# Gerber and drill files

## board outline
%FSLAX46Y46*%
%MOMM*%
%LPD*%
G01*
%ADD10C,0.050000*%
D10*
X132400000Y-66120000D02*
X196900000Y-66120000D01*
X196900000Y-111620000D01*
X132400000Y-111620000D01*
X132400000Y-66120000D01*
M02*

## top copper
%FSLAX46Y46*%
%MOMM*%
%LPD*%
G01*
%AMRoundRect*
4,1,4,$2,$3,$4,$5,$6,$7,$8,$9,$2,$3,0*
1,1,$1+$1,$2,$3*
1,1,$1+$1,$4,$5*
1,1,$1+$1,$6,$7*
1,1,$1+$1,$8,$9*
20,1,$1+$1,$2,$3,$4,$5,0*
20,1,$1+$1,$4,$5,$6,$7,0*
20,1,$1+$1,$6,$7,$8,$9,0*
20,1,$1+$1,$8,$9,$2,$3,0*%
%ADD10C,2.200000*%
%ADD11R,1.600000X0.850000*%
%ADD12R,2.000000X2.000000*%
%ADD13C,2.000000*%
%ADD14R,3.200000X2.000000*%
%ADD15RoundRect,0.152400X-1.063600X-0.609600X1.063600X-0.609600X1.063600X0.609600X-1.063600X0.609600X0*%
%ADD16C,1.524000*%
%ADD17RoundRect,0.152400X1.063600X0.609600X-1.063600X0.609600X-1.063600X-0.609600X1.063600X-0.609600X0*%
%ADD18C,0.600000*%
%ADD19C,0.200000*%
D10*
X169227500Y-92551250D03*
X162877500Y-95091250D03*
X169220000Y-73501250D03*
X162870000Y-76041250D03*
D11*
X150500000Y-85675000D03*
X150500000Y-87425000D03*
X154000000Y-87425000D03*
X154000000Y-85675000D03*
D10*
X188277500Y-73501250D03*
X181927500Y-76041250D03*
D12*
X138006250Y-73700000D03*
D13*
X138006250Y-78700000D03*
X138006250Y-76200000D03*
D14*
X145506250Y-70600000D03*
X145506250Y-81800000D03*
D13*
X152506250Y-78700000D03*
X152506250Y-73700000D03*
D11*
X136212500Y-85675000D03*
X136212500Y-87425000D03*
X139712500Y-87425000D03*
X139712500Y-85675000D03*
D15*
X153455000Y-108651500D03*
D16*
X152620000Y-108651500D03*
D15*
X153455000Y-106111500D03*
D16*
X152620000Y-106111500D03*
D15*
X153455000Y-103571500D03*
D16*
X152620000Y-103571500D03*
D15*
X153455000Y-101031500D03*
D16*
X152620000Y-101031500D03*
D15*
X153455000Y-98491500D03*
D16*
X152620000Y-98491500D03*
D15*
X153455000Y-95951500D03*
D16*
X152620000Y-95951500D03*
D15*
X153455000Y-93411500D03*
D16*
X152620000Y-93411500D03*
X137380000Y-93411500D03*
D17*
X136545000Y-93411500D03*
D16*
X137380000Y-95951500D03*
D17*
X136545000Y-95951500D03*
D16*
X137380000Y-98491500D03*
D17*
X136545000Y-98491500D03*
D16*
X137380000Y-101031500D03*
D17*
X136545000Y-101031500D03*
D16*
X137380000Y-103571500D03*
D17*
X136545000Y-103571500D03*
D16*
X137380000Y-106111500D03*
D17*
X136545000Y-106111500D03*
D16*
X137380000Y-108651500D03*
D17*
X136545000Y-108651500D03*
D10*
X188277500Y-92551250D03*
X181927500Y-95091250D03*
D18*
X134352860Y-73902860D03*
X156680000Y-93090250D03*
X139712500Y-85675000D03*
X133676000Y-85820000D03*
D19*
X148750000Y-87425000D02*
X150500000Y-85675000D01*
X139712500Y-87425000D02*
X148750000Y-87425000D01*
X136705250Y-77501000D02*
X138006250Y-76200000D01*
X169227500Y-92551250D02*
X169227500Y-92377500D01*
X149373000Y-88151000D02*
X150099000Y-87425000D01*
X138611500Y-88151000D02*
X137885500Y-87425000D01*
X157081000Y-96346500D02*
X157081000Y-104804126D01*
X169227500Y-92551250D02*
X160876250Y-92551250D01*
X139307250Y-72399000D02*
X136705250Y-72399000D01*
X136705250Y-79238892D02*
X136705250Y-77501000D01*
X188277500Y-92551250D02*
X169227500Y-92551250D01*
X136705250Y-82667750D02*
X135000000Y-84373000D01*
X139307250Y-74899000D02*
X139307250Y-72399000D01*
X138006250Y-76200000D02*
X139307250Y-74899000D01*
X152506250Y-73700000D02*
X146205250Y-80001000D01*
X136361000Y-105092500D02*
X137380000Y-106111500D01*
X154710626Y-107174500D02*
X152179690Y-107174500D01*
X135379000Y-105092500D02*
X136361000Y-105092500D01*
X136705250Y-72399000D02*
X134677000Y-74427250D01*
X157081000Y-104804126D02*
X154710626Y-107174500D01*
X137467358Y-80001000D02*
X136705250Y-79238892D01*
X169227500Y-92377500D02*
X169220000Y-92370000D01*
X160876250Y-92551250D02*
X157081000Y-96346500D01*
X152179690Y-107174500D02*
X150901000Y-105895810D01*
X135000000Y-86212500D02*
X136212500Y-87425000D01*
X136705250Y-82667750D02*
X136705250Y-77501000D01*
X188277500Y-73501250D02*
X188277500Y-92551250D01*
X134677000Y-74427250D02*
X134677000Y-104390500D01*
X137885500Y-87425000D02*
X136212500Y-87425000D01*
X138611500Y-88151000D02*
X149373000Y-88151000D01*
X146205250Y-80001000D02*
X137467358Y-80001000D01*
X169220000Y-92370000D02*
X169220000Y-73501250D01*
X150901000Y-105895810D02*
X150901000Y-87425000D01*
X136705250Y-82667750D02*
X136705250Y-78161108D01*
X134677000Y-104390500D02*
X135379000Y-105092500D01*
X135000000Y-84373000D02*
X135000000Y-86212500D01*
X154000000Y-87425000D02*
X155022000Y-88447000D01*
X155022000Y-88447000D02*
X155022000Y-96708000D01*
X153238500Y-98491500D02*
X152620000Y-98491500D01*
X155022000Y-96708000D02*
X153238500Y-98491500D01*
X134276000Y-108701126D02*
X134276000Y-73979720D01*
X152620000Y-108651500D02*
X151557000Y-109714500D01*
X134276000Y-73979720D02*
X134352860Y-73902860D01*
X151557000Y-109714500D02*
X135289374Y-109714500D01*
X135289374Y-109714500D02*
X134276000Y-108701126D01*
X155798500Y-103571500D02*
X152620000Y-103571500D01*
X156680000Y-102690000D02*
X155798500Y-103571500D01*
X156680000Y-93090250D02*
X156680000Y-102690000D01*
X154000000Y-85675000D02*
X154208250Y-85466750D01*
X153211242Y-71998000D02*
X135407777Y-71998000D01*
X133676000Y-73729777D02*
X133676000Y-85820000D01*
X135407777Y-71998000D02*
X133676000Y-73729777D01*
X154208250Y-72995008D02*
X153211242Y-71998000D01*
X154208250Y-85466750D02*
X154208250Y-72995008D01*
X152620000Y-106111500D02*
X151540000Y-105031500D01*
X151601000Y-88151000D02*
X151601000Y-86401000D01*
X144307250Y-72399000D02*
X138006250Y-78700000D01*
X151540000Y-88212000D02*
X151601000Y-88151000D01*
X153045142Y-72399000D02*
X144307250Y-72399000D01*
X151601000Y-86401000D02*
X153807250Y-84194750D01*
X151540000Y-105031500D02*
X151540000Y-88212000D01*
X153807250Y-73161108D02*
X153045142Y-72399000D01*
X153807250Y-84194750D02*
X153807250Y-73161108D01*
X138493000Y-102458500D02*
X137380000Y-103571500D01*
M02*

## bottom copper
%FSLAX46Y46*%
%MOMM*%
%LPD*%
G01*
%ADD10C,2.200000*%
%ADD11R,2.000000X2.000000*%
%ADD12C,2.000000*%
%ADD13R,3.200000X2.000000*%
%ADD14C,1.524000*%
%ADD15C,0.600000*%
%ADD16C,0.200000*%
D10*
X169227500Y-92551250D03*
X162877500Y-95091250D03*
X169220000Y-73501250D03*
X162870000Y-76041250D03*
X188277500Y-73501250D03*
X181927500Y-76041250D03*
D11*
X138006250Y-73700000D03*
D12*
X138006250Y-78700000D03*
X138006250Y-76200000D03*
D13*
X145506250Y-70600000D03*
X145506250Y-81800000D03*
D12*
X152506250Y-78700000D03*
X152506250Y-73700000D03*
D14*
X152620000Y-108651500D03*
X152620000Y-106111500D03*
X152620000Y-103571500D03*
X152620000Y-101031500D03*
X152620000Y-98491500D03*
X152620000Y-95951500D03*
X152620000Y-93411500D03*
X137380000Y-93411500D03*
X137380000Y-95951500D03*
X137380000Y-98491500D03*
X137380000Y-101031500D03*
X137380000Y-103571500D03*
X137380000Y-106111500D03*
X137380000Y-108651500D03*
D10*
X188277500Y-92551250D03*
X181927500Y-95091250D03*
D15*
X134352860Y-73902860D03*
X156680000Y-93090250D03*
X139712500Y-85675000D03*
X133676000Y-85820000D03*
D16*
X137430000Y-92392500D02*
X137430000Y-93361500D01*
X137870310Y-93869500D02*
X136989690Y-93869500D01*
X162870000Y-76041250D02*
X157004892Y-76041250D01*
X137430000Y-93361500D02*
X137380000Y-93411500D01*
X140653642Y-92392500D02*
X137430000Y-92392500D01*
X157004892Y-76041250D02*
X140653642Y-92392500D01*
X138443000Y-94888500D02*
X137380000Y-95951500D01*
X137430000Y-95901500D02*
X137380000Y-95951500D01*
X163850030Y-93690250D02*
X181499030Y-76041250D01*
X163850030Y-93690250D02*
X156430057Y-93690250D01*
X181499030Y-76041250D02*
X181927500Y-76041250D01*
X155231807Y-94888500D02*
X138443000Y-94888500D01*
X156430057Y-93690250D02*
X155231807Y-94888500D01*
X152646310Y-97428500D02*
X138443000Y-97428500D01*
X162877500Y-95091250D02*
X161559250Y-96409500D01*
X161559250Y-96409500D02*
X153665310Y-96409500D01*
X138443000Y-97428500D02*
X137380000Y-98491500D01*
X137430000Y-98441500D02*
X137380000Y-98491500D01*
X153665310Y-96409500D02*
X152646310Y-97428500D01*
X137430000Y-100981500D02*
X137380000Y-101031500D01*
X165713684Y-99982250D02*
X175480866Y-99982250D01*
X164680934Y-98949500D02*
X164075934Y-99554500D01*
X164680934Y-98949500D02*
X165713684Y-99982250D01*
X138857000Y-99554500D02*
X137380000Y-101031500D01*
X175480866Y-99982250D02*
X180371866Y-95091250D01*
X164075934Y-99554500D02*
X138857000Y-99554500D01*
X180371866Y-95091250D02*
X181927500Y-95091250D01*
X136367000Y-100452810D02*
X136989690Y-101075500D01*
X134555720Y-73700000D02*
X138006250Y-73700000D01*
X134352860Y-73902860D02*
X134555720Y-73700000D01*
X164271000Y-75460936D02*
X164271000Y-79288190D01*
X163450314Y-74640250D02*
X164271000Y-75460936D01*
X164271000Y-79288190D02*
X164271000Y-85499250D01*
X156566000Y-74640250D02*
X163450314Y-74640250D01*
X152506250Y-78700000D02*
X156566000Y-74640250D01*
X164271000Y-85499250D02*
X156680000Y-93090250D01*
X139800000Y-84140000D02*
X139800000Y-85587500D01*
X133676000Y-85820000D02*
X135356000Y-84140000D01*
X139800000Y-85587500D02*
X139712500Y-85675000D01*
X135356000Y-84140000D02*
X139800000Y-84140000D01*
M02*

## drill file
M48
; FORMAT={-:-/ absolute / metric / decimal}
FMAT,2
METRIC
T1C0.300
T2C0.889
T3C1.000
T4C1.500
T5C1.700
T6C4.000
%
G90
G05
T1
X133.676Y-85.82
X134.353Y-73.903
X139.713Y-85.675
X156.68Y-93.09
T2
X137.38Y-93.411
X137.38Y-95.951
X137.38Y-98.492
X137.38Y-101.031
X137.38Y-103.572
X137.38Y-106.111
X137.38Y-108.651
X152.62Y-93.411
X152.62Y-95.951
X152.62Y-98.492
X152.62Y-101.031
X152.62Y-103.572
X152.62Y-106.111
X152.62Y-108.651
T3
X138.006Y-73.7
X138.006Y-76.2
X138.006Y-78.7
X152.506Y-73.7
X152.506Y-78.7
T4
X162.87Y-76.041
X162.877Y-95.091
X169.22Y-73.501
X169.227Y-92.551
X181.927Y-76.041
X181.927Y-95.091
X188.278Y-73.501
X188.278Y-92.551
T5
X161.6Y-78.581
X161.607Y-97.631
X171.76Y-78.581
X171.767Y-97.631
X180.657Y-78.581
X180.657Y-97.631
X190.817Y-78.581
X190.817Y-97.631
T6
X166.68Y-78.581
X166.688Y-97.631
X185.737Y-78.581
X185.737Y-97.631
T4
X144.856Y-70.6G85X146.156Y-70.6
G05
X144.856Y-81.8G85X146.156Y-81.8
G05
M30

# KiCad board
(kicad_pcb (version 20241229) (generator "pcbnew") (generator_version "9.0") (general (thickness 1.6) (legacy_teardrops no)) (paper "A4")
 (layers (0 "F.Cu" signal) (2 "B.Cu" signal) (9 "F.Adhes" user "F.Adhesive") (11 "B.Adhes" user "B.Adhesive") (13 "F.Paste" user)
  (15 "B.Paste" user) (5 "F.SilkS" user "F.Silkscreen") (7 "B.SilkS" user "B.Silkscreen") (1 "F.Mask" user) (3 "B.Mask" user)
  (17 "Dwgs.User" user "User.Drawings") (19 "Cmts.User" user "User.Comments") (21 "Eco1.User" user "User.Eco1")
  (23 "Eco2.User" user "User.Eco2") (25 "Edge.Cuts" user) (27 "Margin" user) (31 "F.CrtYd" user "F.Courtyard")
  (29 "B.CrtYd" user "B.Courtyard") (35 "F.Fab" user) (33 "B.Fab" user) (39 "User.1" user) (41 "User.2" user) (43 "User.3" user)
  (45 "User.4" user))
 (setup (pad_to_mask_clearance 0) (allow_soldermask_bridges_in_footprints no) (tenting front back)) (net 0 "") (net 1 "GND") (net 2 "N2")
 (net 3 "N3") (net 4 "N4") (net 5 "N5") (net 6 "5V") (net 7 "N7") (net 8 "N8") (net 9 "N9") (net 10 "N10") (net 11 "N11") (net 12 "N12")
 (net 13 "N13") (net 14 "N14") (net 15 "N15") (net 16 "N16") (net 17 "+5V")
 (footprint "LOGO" (layer "F.Cu") (at 140.493481 67.83475)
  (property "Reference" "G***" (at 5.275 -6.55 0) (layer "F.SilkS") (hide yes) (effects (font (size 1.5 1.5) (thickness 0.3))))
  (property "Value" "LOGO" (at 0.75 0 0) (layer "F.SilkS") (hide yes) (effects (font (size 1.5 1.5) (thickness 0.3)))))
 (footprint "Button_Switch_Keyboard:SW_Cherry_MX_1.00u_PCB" (layer "F.Cu") (at 169.2275 92.55125)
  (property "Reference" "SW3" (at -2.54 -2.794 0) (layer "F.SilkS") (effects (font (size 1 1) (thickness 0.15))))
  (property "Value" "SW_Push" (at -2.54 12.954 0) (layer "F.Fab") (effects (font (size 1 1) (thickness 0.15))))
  (pad "" np_thru_hole circle (at -7.62 5.08) (size 1.7 1.7) (drill 1.7) (layers "*.Cu" "*.Mask"))
  (pad "" np_thru_hole circle (at -2.54 5.08) (size 4 4) (drill 4) (layers "*.Cu" "*.Mask"))
  (pad "" np_thru_hole circle (at 2.54 5.08) (size 1.7 1.7) (drill 1.7) (layers "*.Cu" "*.Mask"))
  (pad "1" thru_hole circle (at 0 0) (size 2.2 2.2) (drill 1.5) (layers "*.Cu" "*.Mask") (remove_unused_layers no) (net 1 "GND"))
  (pad "2" thru_hole circle (at -6.35 2.54) (size 2.2 2.2) (drill 1.5) (layers "*.Cu" "*.Mask") (remove_unused_layers no) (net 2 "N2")))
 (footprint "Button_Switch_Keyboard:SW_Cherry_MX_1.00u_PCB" (layer "F.Cu") (at 169.22 73.50125)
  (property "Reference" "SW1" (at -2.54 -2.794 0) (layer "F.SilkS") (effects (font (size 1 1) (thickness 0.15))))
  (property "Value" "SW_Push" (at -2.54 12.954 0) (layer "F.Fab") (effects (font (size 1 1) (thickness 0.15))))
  (pad "" np_thru_hole circle (at -7.62 5.08) (size 1.7 1.7) (drill 1.7) (layers "*.Cu" "*.Mask"))
  (pad "" np_thru_hole circle (at -2.54 5.08) (size 4 4) (drill 4) (layers "*.Cu" "*.Mask"))
  (pad "" np_thru_hole circle (at 2.54 5.08) (size 1.7 1.7) (drill 1.7) (layers "*.Cu" "*.Mask"))
  (pad "1" thru_hole circle (at 0 0) (size 2.2 2.2) (drill 1.5) (layers "*.Cu" "*.Mask") (remove_unused_layers no) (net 1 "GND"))
  (pad "2" thru_hole circle (at -6.35 2.54) (size 2.2 2.2) (drill 1.5) (layers "*.Cu" "*.Mask") (remove_unused_layers no) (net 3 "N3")))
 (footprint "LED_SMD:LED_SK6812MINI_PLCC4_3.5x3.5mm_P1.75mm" (layer "F.Cu") (at 152.25 86.55)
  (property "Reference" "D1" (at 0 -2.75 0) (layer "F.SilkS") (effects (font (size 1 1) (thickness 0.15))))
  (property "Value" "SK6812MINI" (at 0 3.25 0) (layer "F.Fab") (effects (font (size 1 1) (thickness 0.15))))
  (pad "1" smd rect (at -1.75 -0.875) (size 1.6 0.85) (layers "F.Cu" "F.Mask" "F.Paste") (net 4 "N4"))
  (pad "2" smd rect (at -1.75 0.875) (size 1.6 0.85) (layers "F.Cu" "F.Mask" "F.Paste") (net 1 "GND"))
  (pad "3" smd rect (at 1.75 0.875) (size 1.6 0.85) (layers "F.Cu" "F.Mask" "F.Paste") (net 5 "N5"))
  (pad "4" smd rect (at 1.75 -0.875) (size 1.6 0.85) (layers "F.Cu" "F.Mask" "F.Paste") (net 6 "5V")))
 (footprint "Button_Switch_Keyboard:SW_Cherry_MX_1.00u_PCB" (layer "F.Cu") (at 188.2775 73.50125)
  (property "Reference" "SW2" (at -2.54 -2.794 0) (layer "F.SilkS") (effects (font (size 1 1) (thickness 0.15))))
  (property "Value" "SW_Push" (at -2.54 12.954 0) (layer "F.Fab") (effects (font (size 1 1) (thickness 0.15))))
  (pad "" np_thru_hole circle (at -7.62 5.08) (size 1.7 1.7) (drill 1.7) (layers "*.Cu" "*.Mask"))
  (pad "" np_thru_hole circle (at -2.54 5.08) (size 4 4) (drill 4) (layers "*.Cu" "*.Mask"))
  (pad "" np_thru_hole circle (at 2.54 5.08) (size 1.7 1.7) (drill 1.7) (layers "*.Cu" "*.Mask"))
  (pad "1" thru_hole circle (at 0 0) (size 2.2 2.2) (drill 1.5) (layers "*.Cu" "*.Mask") (remove_unused_layers no) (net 1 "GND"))
  (pad "2" thru_hole circle (at -6.35 2.54) (size 2.2 2.2) (drill 1.5) (layers "*.Cu" "*.Mask") (remove_unused_layers no) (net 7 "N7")))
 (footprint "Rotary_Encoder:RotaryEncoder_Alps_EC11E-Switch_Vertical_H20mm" (layer "F.Cu") (at 138.00625 73.7)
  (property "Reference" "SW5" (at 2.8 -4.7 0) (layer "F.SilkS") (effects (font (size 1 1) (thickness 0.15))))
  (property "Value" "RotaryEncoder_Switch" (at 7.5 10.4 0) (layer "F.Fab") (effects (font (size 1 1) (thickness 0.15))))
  (pad "A" thru_hole rect (at 0 0) (size 2 2) (drill 1) (layers "*.Cu" "*.Mask") (remove_unused_layers no) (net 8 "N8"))
  (pad "B" thru_hole circle (at 0 5) (size 2 2) (drill 1) (layers "*.Cu" "*.Mask") (remove_unused_layers no) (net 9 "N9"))
  (pad "C" thru_hole circle (at 0 2.5) (size 2 2) (drill 1) (layers "*.Cu" "*.Mask") (remove_unused_layers no) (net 1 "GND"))
  (pad "MP" thru_hole rect (at 7.5 -3.1) (size 3.2 2) (drill oval 2.8 1.5) (layers "*.Cu" "*.Mask") (remove_unused_layers no))
  (pad "MP" thru_hole rect (at 7.5 8.1) (size 3.2 2) (drill oval 2.8 1.5) (layers "*.Cu" "*.Mask") (remove_unused_layers no))
  (pad "S1" thru_hole circle (at 14.5 5) (size 2 2) (drill 1) (layers "*.Cu" "*.Mask") (remove_unused_layers no) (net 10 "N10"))
  (pad "S2" thru_hole circle (at 14.5 0) (size 2 2) (drill 1) (layers "*.Cu" "*.Mask") (remove_unused_layers no) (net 1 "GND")))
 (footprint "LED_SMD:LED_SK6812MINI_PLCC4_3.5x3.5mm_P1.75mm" (layer "F.Cu") (at 137.9625 86.55)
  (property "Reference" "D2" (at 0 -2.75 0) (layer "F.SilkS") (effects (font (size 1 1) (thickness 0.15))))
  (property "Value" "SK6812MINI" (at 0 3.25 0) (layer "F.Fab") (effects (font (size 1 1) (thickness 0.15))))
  (pad "1" smd rect (at -1.75 -0.875) (size 1.6 0.85) (layers "F.Cu" "F.Mask" "F.Paste") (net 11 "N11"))
  (pad "2" smd rect (at -1.75 0.875) (size 1.6 0.85) (layers "F.Cu" "F.Mask" "F.Paste") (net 1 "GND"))
  (pad "3" smd rect (at 1.75 0.875) (size 1.6 0.85) (layers "F.Cu" "F.Mask" "F.Paste") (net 4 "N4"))
  (pad "4" smd rect (at 1.75 -0.875) (size 1.6 0.85) (layers "F.Cu" "F.Mask" "F.Paste") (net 6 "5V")))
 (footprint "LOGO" (layer "F.Cu") (at 189.413481 67.69475)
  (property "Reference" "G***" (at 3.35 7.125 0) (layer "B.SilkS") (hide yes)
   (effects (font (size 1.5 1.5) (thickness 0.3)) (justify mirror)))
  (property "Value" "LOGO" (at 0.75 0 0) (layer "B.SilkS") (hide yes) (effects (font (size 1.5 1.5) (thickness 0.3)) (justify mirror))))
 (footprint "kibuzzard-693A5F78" (layer "F.Cu") (at 176.275 108.05 180)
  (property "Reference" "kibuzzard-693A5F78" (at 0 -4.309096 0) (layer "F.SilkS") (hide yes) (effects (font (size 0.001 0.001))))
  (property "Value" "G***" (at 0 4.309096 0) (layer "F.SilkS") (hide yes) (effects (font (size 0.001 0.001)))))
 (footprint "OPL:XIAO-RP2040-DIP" (layer "F.Cu") (at 145 101.0315 180)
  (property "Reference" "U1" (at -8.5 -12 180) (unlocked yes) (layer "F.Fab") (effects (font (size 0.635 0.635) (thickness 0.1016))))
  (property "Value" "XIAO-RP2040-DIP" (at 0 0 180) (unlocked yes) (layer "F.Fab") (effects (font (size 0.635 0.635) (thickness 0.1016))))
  (pad "1" smd roundrect (at -8.455 -7.62) (size 2.432 1.524) (layers "F.Cu" "F.Mask") (roundrect_rratio 0.1) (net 8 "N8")
   (thermal_bridge_angle 45))
  (pad "1" thru_hole circle (at -7.62 -7.62) (size 1.524 1.524) (drill 0.889) (layers "*.Cu" "*.Mask") (remove_unused_layers no)
   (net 8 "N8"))
  (pad "2" smd roundrect (at -8.455 -5.08) (size 2.432 1.524) (layers "F.Cu" "F.Mask") (roundrect_rratio 0.1) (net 9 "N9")
   (thermal_bridge_angle 45))
  (pad "2" thru_hole circle (at -7.62 -5.08) (size 1.524 1.524) (drill 0.889) (layers "*.Cu" "*.Mask") (remove_unused_layers no)
   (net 9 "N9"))
  (pad "3" smd roundrect (at -8.455 -2.54) (size 2.432 1.524) (layers "F.Cu" "F.Mask") (roundrect_rratio 0.1) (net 10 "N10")
   (thermal_bridge_angle 45))
  (pad "3" thru_hole circle (at -7.62 -2.54) (size 1.524 1.524) (drill 0.889) (layers "*.Cu" "*.Mask") (remove_unused_layers no)
   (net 10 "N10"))
  (pad "4" smd roundrect (at -8.455 0) (size 2.432 1.524) (layers "F.Cu" "F.Mask") (roundrect_rratio 0.1) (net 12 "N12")
   (thermal_bridge_angle 45))
  (pad "4" thru_hole circle (at -7.62 0) (size 1.524 1.524) (drill 0.889) (layers "*.Cu" "*.Mask") (remove_unused_layers no) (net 12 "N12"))
  (pad "5" smd roundrect (at -8.455 2.54) (size 2.432 1.524) (layers "F.Cu" "F.Mask") (roundrect_rratio 0.1) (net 5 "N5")
   (thermal_bridge_angle 45))
  (pad "5" thru_hole circle (at -7.62 2.54) (size 1.524 1.524) (drill 0.889) (layers "*.Cu" "*.Mask") (remove_unused_layers no) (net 5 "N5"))
  (pad "6" smd roundrect (at -8.455 5.08) (size 2.432 1.524) (layers "F.Cu" "F.Mask") (roundrect_rratio 0.1) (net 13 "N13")
   (thermal_bridge_angle 45))
  (pad "6" thru_hole circle (at -7.62 5.08) (size 1.524 1.524) (drill 0.889) (layers "*.Cu" "*.Mask") (remove_unused_layers no)
   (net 13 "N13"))
  (pad "7" smd roundrect (at -8.455 7.62) (size 2.432 1.524) (layers "F.Cu" "F.Mask") (roundrect_rratio 0.1) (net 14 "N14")
   (thermal_bridge_angle 45))
  (pad "7" thru_hole circle (at -7.62 7.62) (size 1.524 1.524) (drill 0.889) (layers "*.Cu" "*.Mask") (remove_unused_layers no)
   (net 14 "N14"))
  (pad "8" thru_hole circle (at 7.62 7.62 180) (size 1.524 1.524) (drill 0.889) (layers "*.Cu" "*.Mask") (remove_unused_layers no)
   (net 3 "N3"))
  (pad "8" smd roundrect (at 8.455 7.62 180) (size 2.432 1.524) (layers "F.Cu" "F.Mask") (roundrect_rratio 0.1) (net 3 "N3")
   (thermal_bridge_angle 45))
  (pad "9" thru_hole circle (at 7.62 5.08 180) (size 1.524 1.524) (drill 0.889) (layers "*.Cu" "*.Mask") (remove_unused_layers no)
   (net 7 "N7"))
  (pad "9" smd roundrect (at 8.455 5.08 180) (size 2.432 1.524) (layers "F.Cu" "F.Mask") (roundrect_rratio 0.1) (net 7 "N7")
   (thermal_bridge_angle 45))
  (pad "10" thru_hole circle (at 7.62 2.54 180) (size 1.524 1.524) (drill 0.889) (layers "*.Cu" "*.Mask") (remove_unused_layers no)
   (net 2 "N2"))
  (pad "10" smd roundrect (at 8.455 2.54 180) (size 2.432 1.524) (layers "F.Cu" "F.Mask") (roundrect_rratio 0.1) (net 2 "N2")
   (thermal_bridge_angle 45))
  (pad "11" thru_hole circle (at 7.62 0 180) (size 1.524 1.524) (drill 0.889) (layers "*.Cu" "*.Mask") (remove_unused_layers no)
   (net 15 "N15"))
  (pad "11" smd roundrect (at 8.455 0 180) (size 2.432 1.524) (layers "F.Cu" "F.Mask") (roundrect_rratio 0.1) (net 15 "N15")
   (thermal_bridge_angle 45))
  (pad "12" thru_hole circle (at 7.62 -2.54 180) (size 1.524 1.524) (drill 0.889) (layers "*.Cu" "*.Mask") (remove_unused_layers no)
   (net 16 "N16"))
  (pad "12" smd roundrect (at 8.455 -2.54 180) (size 2.432 1.524) (layers "F.Cu" "F.Mask") (roundrect_rratio 0.1) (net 16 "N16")
   (thermal_bridge_angle 45))
  (pad "13" thru_hole circle (at 7.62 -5.08 180) (size 1.524 1.524) (drill 0.889) (layers "*.Cu" "*.Mask") (remove_unused_layers no)
   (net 1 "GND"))
  (pad "13" smd roundrect (at 8.455 -5.08 180) (size 2.432 1.524) (layers "F.Cu" "F.Mask") (roundrect_rratio 0.1) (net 1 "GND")
   (thermal_bridge_angle 45))
  (pad "14" thru_hole circle (at 7.62 -7.62 180) (size 1.524 1.524) (drill 0.889) (layers "*.Cu" "*.Mask") (remove_unused_layers no)
   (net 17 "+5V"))
  (pad "14" smd roundrect (at 8.455 -7.62 180) (size 2.432 1.524) (layers "F.Cu" "F.Mask") (roundrect_rratio 0.1) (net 17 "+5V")
   (thermal_bridge_angle 45)))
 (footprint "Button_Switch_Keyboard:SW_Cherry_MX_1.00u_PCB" (layer "F.Cu") (at 188.2775 92.55125)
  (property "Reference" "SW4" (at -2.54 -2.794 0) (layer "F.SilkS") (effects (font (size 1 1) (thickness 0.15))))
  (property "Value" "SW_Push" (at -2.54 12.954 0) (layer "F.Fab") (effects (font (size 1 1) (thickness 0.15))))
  (pad "" np_thru_hole circle (at -7.62 5.08) (size 1.7 1.7) (drill 1.7) (layers "*.Cu" "*.Mask"))
  (pad "" np_thru_hole circle (at -2.54 5.08) (size 4 4) (drill 4) (layers "*.Cu" "*.Mask"))
  (pad "" np_thru_hole circle (at 2.54 5.08) (size 1.7 1.7) (drill 1.7) (layers "*.Cu" "*.Mask"))
  (pad "1" thru_hole circle (at 0 0) (size 2.2 2.2) (drill 1.5) (layers "*.Cu" "*.Mask") (remove_unused_layers no) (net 1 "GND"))
  (pad "2" thru_hole circle (at -6.35 2.54) (size 2.2 2.2) (drill 1.5) (layers "*.Cu" "*.Mask") (remove_unused_layers no) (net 15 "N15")))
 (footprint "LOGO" (layer "B.Cu") (at 187.645571 108.957432 180)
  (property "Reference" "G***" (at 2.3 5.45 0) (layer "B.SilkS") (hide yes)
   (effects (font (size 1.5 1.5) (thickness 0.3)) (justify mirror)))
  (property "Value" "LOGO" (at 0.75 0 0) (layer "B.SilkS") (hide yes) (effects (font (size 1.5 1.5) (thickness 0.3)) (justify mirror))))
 (gr_rect (start 132.4 66.12) (end 196.9 111.62) (stroke (width 0.05) (type solid)) (fill no) (layer "Edge.Cuts"))
 (segment (start 148.75 87.425) (end 150.5 85.675) (width 0.2) (layer "F.Cu") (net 4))
 (segment (start 139.7125 87.425) (end 148.75 87.425) (width 0.2) (layer "F.Cu") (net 4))
 (segment (start 136.70525 77.501) (end 138.00625 76.2) (width 0.2) (layer "F.Cu") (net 1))
 (segment (start 169.2275 92.55125) (end 169.2275 92.3775) (width 0.2) (layer "F.Cu") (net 1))
 (segment (start 149.373 88.151) (end 150.099 87.425) (width 0.2) (layer "F.Cu") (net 1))
 (segment (start 138.6115 88.151) (end 137.8855 87.425) (width 0.2) (layer "F.Cu") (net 1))
 (segment (start 157.081 96.3465) (end 157.081 104.804126) (width 0.2) (layer "F.Cu") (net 1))
 (segment (start 169.2275 92.55125) (end 160.87625 92.55125) (width 0.2) (layer "F.Cu") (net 1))
 (segment (start 139.30725 72.399) (end 136.70525 72.399) (width 0.2) (layer "F.Cu") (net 1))
 (segment (start 136.70525 79.238892) (end 136.70525 77.501) (width 0.2) (layer "F.Cu") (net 1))
 (segment (start 188.2775 92.55125) (end 169.2275 92.55125) (width 0.2) (layer "F.Cu") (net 1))
 (segment (start 136.70525 82.66775) (end 135 84.373) (width 0.2) (layer "F.Cu") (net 1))
 (segment (start 139.30725 74.899) (end 139.30725 72.399) (width 0.2) (layer "F.Cu") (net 1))
 (segment (start 138.00625 76.2) (end 139.30725 74.899) (width 0.2) (layer "F.Cu") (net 1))
 (segment (start 152.50625 73.7) (end 146.20525 80.001) (width 0.2) (layer "F.Cu") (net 1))
 (segment (start 136.361 105.0925) (end 137.38 106.1115) (width 0.2) (layer "F.Cu") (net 1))
 (segment (start 154.710626 107.1745) (end 152.17969 107.1745) (width 0.2) (layer "F.Cu") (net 1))
 (segment (start 135.379 105.0925) (end 136.361 105.0925) (width 0.2) (layer "F.Cu") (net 1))
 (segment (start 136.70525 72.399) (end 134.677 74.42725) (width 0.2) (layer "F.Cu") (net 1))
 (segment (start 157.081 104.804126) (end 154.710626 107.1745) (width 0.2) (layer "F.Cu") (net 1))
 (segment (start 137.467358 80.001) (end 136.70525 79.238892) (width 0.2) (layer "F.Cu") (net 1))
 (segment (start 169.2275 92.3775) (end 169.22 92.37) (width 0.2) (layer "F.Cu") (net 1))
 (segment (start 160.87625 92.55125) (end 157.081 96.3465) (width 0.2) (layer "F.Cu") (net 1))
 (segment (start 152.17969 107.1745) (end 150.901 105.89581) (width 0.2) (layer "F.Cu") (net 1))
 (segment (start 135 86.2125) (end 136.2125 87.425) (width 0.2) (layer "F.Cu") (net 1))
 (segment (start 136.70525 82.66775) (end 136.70525 77.501) (width 0.2) (layer "F.Cu") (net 1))
 (segment (start 188.2775 73.50125) (end 188.2775 92.55125) (width 0.2) (layer "F.Cu") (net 1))
 (segment (start 134.677 74.42725) (end 134.677 104.3905) (width 0.2) (layer "F.Cu") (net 1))
 (segment (start 137.8855 87.425) (end 136.2125 87.425) (width 0.2) (layer "F.Cu") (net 1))
 (segment (start 138.6115 88.151) (end 149.373 88.151) (width 0.2) (layer "F.Cu") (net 1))
 (segment (start 146.20525 80.001) (end 137.467358 80.001) (width 0.2) (layer "F.Cu") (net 1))
 (segment (start 169.22 92.37) (end 169.22 73.50125) (width 0.2) (layer "F.Cu") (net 1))
 (segment (start 150.901 105.89581) (end 150.901 87.425) (width 0.2) (layer "F.Cu") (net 1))
 (segment (start 136.70525 82.66775) (end 136.70525 78.161108) (width 0.2) (layer "F.Cu") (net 1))
 (segment (start 134.677 104.3905) (end 135.379 105.0925) (width 0.2) (layer "F.Cu") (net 1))
 (segment (start 135 84.373) (end 135 86.2125) (width 0.2) (layer "F.Cu") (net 1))
 (segment (start 154 87.425) (end 155.022 88.447) (width 0.2) (layer "F.Cu") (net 5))
 (segment (start 155.022 88.447) (end 155.022 96.708) (width 0.2) (layer "F.Cu") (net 5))
 (segment (start 153.2385 98.4915) (end 152.62 98.4915) (width 0.2) (layer "F.Cu") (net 5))
 (segment (start 155.022 96.708) (end 153.2385 98.4915) (width 0.2) (layer "F.Cu") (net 5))
 (segment (start 137.43 92.3925) (end 137.43 93.3615) (width 0.2) (layer "B.Cu") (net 3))
 (segment (start 137.87031 93.8695) (end 136.98969 93.8695) (width 0.2) (layer "B.Cu") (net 3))
 (segment (start 162.87 76.04125) (end 157.004892 76.04125) (width 0.2) (layer "B.Cu") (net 3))
 (segment (start 137.43 93.3615) (end 137.38 93.4115) (width 0.2) (layer "B.Cu") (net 3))
 (segment (start 140.653642 92.3925) (end 137.43 92.3925) (width 0.2) (layer "B.Cu") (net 3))
 (segment (start 157.004892 76.04125) (end 140.653642 92.3925) (width 0.2) (layer "B.Cu") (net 3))
 (segment (start 138.443 94.8885) (end 137.38 95.9515) (width 0.2) (layer "B.Cu") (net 7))
 (segment (start 137.43 95.9015) (end 137.38 95.9515) (width 0.2) (layer "B.Cu") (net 7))
 (segment (start 163.85003 93.69025) (end 181.49903 76.04125) (width 0.2) (layer "B.Cu") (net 7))
 (segment (start 163.85003 93.69025) (end 156.430057 93.69025) (width 0.2) (layer "B.Cu") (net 7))
 (segment (start 181.49903 76.04125) (end 181.9275 76.04125) (width 0.2) (layer "B.Cu") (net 7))
 (segment (start 155.231807 94.8885) (end 138.443 94.8885) (width 0.2) (layer "B.Cu") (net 7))
 (segment (start 156.430057 93.69025) (end 155.231807 94.8885) (width 0.2) (layer "B.Cu") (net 7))
 (segment (start 152.64631 97.4285) (end 138.443 97.4285) (width 0.2) (layer "B.Cu") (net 2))
 (segment (start 162.8775 95.09125) (end 161.55925 96.4095) (width 0.2) (layer "B.Cu") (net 2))
 (segment (start 161.55925 96.4095) (end 153.66531 96.4095) (width 0.2) (layer "B.Cu") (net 2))
 (segment (start 138.443 97.4285) (end 137.38 98.4915) (width 0.2) (layer "B.Cu") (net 2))
 (segment (start 137.43 98.4415) (end 137.38 98.4915) (width 0.2) (layer "B.Cu") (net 2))
 (segment (start 153.66531 96.4095) (end 152.64631 97.4285) (width 0.2) (layer "B.Cu") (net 2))
 (segment (start 137.43 100.9815) (end 137.38 101.0315) (width 0.2) (layer "B.Cu") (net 15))
 (segment (start 165.713684 99.98225) (end 175.480866 99.98225) (width 0.2) (layer "B.Cu") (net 15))
 (segment (start 164.680934 98.9495) (end 164.075934 99.5545) (width 0.2) (layer "B.Cu") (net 15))
 (segment (start 164.680934 98.9495) (end 165.713684 99.98225) (width 0.2) (layer "B.Cu") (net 15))
 (segment (start 138.857 99.5545) (end 137.38 101.0315) (width 0.2) (layer "B.Cu") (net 15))
 (segment (start 175.480866 99.98225) (end 180.371866 95.09125) (width 0.2) (layer "B.Cu") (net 15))
 (segment (start 164.075934 99.5545) (end 138.857 99.5545) (width 0.2) (layer "B.Cu") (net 15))
 (segment (start 180.371866 95.09125) (end 181.9275 95.09125) (width 0.2) (layer "B.Cu") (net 15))
 (segment (start 136.367 100.45281) (end 136.98969 101.0755) (width 0.2) (layer "B.Cu") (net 15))
 (segment (start 134.276 108.701126) (end 134.276 73.97972) (width 0.2) (layer "F.Cu") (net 8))
 (segment (start 152.62 108.6515) (end 151.557 109.7145) (width 0.2) (layer "F.Cu") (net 8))
 (segment (start 134.276 73.97972) (end 134.35286 73.90286) (width 0.2) (layer "F.Cu") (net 8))
 (segment (start 151.557 109.7145) (end 135.289374 109.7145) (width 0.2) (layer "F.Cu") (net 8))
 (segment (start 135.289374 109.7145) (end 134.276 108.701126) (width 0.2) (layer "F.Cu") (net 8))
 (via (at 134.35286 73.90286) (size 0.6) (drill 0.3) (layers "F.Cu" "B.Cu") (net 8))
 (segment (start 134.55572 73.7) (end 138.00625 73.7) (width 0.2) (layer "B.Cu") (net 8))
 (segment (start 134.35286 73.90286) (end 134.55572 73.7) (width 0.2) (layer "B.Cu") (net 8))
 (segment (start 155.7985 103.5715) (end 152.62 103.5715) (width 0.2) (layer "F.Cu") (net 10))
 (segment (start 156.68 102.69) (end 155.7985 103.5715) (width 0.2) (layer "F.Cu") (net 10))
 (segment (start 156.68 93.09025) (end 156.68 102.69) (width 0.2) (layer "F.Cu") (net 10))
 (via (at 156.68 93.09025) (size 0.6) (drill 0.3) (layers "F.Cu" "B.Cu") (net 10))
 (segment (start 164.271 75.460936) (end 164.271 79.28819) (width 0.2) (layer "B.Cu") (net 10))
 (segment (start 163.450314 74.64025) (end 164.271 75.460936) (width 0.2) (layer "B.Cu") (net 10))
 (segment (start 164.271 79.28819) (end 164.271 85.49925) (width 0.2) (layer "B.Cu") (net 10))
 (segment (start 156.566 74.64025) (end 163.450314 74.64025) (width 0.2) (layer "B.Cu") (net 10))
 (segment (start 152.50625 78.7) (end 156.566 74.64025) (width 0.2) (layer "B.Cu") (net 10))
 (segment (start 164.271 85.49925) (end 156.68 93.09025) (width 0.2) (layer "B.Cu") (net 10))
 (segment (start 154 85.675) (end 154.20825 85.46675) (width 0.2) (layer "F.Cu") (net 6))
 (segment (start 153.211242 71.998) (end 135.407777 71.998) (width 0.2) (layer "F.Cu") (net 6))
 (segment (start 133.676 73.729777) (end 133.676 85.82) (width 0.2) (layer "F.Cu") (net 6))
 (segment (start 135.407777 71.998) (end 133.676 73.729777) (width 0.2) (layer "F.Cu") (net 6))
 (segment (start 154.20825 72.995008) (end 153.211242 71.998) (width 0.2) (layer "F.Cu") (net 6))
 (segment (start 154.20825 85.46675) (end 154.20825 72.995008) (width 0.2) (layer "F.Cu") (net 6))
 (via (at 139.7125 85.675) (size 0.6) (drill 0.3) (layers "F.Cu" "B.Cu") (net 6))
 (via (at 133.676 85.82) (size 0.6) (drill 0.3) (layers "F.Cu" "B.Cu") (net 6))
 (segment (start 139.8 84.14) (end 139.8 85.5875) (width 0.2) (layer "B.Cu") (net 6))
 (segment (start 133.676 85.82) (end 135.356 84.14) (width 0.2) (layer "B.Cu") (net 6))
 (segment (start 139.8 85.5875) (end 139.7125 85.675) (width 0.2) (layer "B.Cu") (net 6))
 (segment (start 135.356 84.14) (end 139.8 84.14) (width 0.2) (layer "B.Cu") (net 6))
 (segment (start 152.62 106.1115) (end 151.54 105.0315) (width 0.2) (layer "F.Cu") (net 9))
 (segment (start 151.601 88.151) (end 151.601 86.401) (width 0.2) (layer "F.Cu") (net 9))
 (segment (start 144.30725 72.399) (end 138.00625 78.7) (width 0.2) (layer "F.Cu") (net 9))
 (segment (start 151.54 88.212) (end 151.601 88.151) (width 0.2) (layer "F.Cu") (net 9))
 (segment (start 153.045142 72.399) (end 144.30725 72.399) (width 0.2) (layer "F.Cu") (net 9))
 (segment (start 151.601 86.401) (end 153.80725 84.19475) (width 0.2) (layer "F.Cu") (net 9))
 (segment (start 151.54 105.0315) (end 151.54 88.212) (width 0.2) (layer "F.Cu") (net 9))
 (segment (start 153.80725 73.161108) (end 153.045142 72.399) (width 0.2) (layer "F.Cu") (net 9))
 (segment (start 153.80725 84.19475) (end 153.80725 73.161108) (width 0.2) (layer "F.Cu") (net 9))
 (segment (start 138.493 102.4585) (end 137.38 103.5715) (width 0.2) (layer "F.Cu") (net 16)))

